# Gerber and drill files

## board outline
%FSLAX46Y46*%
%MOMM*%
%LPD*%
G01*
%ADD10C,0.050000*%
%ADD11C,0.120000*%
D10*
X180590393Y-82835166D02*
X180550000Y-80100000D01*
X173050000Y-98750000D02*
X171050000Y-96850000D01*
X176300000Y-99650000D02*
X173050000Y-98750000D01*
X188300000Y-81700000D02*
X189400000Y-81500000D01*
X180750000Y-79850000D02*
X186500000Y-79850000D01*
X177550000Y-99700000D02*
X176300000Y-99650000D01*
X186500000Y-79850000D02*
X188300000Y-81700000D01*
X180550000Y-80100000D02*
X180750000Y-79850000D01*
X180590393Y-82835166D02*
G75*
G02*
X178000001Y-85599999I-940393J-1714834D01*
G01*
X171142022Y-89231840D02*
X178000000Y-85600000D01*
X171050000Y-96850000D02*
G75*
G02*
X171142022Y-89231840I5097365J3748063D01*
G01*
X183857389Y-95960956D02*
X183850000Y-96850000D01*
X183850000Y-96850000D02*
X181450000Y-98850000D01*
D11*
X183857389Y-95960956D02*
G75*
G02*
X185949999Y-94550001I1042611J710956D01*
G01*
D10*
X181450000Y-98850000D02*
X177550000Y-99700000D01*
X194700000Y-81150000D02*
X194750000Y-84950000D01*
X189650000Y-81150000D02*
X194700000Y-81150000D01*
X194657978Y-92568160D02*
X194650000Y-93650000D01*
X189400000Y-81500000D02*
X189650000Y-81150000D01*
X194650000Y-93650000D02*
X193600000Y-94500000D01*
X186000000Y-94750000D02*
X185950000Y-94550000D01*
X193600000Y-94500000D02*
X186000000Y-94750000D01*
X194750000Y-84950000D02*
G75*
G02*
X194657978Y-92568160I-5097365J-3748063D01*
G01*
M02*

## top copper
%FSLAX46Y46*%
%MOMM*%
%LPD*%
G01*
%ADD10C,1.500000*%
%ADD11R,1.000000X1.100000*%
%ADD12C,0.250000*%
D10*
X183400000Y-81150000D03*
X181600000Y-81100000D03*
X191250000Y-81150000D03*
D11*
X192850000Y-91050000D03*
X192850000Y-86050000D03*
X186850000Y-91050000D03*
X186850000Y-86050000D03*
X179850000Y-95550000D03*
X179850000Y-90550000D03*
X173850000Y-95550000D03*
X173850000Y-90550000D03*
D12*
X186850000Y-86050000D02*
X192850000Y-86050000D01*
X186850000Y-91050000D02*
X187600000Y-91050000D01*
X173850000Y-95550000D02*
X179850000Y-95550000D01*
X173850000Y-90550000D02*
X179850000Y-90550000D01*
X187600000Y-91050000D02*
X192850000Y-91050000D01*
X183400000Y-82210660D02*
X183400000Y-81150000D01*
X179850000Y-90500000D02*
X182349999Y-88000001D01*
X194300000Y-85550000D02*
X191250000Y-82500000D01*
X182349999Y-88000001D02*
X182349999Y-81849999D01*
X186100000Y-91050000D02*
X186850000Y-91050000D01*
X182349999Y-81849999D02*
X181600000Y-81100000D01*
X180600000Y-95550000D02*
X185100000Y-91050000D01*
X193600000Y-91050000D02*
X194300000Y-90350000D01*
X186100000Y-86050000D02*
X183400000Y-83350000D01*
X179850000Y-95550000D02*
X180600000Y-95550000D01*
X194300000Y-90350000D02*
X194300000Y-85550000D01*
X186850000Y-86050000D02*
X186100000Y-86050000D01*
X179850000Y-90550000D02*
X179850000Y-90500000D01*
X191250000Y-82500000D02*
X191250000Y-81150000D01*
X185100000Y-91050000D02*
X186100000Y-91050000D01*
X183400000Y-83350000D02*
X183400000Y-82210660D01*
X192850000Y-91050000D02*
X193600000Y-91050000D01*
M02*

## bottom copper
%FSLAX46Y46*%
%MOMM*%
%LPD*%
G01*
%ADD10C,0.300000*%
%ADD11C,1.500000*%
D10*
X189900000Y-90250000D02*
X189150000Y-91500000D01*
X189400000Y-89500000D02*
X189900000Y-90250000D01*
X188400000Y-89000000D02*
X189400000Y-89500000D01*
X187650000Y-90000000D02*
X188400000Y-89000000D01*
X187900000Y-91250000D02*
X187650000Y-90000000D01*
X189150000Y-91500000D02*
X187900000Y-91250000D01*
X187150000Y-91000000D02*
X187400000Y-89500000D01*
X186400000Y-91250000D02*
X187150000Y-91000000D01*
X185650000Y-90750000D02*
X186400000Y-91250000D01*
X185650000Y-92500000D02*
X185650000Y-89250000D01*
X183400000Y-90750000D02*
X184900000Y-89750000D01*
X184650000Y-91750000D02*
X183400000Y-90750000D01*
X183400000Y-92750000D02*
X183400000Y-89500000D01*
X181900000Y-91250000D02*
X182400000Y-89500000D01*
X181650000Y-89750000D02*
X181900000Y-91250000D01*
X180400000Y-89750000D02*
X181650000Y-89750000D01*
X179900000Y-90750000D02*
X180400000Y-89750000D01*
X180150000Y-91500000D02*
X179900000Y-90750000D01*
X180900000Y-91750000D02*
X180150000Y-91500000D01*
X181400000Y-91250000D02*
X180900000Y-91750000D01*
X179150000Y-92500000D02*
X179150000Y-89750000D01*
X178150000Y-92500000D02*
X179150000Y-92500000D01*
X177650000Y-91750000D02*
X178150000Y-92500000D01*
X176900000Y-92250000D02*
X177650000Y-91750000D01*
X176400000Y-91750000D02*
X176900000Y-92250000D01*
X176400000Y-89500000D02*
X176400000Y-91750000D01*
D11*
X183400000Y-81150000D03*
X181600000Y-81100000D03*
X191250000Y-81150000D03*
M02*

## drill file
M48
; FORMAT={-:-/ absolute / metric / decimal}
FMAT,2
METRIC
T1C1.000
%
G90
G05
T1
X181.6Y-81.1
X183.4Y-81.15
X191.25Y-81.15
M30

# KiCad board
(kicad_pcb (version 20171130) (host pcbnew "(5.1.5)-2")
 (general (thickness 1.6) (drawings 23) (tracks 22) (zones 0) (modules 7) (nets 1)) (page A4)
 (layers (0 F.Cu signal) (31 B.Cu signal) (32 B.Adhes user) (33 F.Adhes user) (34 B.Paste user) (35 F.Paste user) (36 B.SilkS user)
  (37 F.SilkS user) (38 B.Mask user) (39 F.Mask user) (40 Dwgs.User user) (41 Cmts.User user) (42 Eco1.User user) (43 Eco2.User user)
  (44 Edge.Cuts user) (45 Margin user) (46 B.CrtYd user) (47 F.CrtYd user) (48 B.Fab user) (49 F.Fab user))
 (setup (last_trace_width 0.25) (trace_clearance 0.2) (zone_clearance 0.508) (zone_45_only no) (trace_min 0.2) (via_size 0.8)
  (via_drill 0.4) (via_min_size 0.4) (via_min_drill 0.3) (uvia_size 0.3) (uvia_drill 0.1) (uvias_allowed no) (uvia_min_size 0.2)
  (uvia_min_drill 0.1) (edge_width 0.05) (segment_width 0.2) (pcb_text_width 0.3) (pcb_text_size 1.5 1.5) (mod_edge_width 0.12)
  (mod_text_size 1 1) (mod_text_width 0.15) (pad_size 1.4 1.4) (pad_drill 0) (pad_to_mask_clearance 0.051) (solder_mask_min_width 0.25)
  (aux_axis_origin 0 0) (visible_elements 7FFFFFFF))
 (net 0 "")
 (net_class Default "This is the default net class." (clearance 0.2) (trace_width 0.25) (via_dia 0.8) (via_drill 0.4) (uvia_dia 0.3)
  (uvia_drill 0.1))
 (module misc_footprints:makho (layer B.Cu) (at 182.9 90.75)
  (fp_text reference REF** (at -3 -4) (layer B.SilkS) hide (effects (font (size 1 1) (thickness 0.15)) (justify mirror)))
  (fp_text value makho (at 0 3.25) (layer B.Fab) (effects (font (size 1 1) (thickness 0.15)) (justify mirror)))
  (fp_line (start 7 -0.5) (end 6.25 0.75) (layer B.Cu) (width 0.3))
  (fp_line (start 6.5 -1.25) (end 7 -0.5) (layer B.Cu) (width 0.3))
  (fp_line (start 5.5 -1.75) (end 6.5 -1.25) (layer B.Cu) (width 0.3))
  (fp_line (start 4.75 -0.75) (end 5.5 -1.75) (layer B.Cu) (width 0.3))
  (fp_line (start 5 0.5) (end 4.75 -0.75) (layer B.Cu) (width 0.3))
  (fp_line (start 6.25 0.75) (end 5 0.5) (layer B.Cu) (width 0.3))
  (fp_line (start 4.25 0.25) (end 4.5 -1.25) (layer B.Cu) (width 0.3))
  (fp_line (start 3.5 0.5) (end 4.25 0.25) (layer B.Cu) (width 0.3))
  (fp_line (start 2.75 0) (end 3.5 0.5) (layer B.Cu) (width 0.3))
  (fp_line (start 2.75 1.75) (end 2.75 -1.5) (layer B.Cu) (width 0.3)) (fp_line (start 0.5 0) (end 2 -1) (layer B.Cu) (width 0.3))
  (fp_line (start 1.75 1) (end 0.5 0) (layer B.Cu) (width 0.3))
  (fp_line (start 0.5 2) (end 0.5 -1.25) (layer B.Cu) (width 0.3))
  (fp_line (start -1 0.5) (end -0.5 -1.25) (layer B.Cu) (width 0.3))
  (fp_line (start -1.25 -1) (end -1 0.5) (layer B.Cu) (width 0.3))
  (fp_line (start -2.5 -1) (end -1.25 -1) (layer B.Cu) (width 0.3))
  (fp_line (start -3 0) (end -2.5 -1) (layer B.Cu) (width 0.3))
  (fp_line (start -2.75 0.75) (end -3 0) (layer B.Cu) (width 0.3))
  (fp_line (start -2 1) (end -2.75 0.75) (layer B.Cu) (width 0.3))
  (fp_line (start -1.5 0.5) (end -2 1) (layer B.Cu) (width 0.3))
  (fp_line (start -3.75 1.75) (end -3.75 -1) (layer B.Cu) (width 0.3))
  (fp_line (start -4.75 1.75) (end -3.75 1.75) (layer B.Cu) (width 0.3))
  (fp_line (start -5.25 1) (end -4.75 1.75) (layer B.Cu) (width 0.3))
  (fp_line (start -6 1.5) (end -5.25 1) (layer B.Cu) (width 0.3))
  (fp_line (start -6.5 1) (end -6 1.5) (layer B.Cu) (width 0.3))
  (fp_line (start -6.5 -1.25) (end -6.5 1) (layer B.Cu) (width 0.3)))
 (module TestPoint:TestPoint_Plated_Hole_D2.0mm (layer F.Cu) (at 183.4 81.15)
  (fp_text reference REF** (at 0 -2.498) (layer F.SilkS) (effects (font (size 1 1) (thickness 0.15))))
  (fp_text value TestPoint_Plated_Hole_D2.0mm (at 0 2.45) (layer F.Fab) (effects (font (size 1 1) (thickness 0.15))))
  (pad 1 thru_hole circle (at 0 0) (size 1.5 1.5) (drill 1) (layers *.Cu *.Mask)))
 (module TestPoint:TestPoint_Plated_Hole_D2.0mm (layer F.Cu) (at 181.6 81.1)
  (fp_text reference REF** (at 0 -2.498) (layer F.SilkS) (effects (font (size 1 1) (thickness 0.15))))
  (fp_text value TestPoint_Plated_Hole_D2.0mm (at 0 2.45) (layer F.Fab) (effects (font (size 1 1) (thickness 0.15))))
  (pad 1 thru_hole circle (at 0 0) (size 1.5 1.5) (drill 1) (layers *.Cu *.Mask)))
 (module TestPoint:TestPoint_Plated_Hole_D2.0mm (layer F.Cu) (at 191.25 81.15)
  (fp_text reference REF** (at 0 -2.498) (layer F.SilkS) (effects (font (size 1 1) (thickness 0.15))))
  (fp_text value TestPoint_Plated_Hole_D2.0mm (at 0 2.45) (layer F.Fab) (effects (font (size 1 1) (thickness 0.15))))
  (pad 1 thru_hole circle (at 0 0) (size 1.5 1.5) (drill 1) (layers *.Cu *.Mask)))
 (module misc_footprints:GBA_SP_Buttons (layer F.Cu) (at 189.85 88.55)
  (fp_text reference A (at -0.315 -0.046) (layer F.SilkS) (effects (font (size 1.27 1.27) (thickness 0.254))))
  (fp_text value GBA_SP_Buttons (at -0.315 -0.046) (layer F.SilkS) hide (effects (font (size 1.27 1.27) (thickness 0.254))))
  (pad 4 smd rect (at 3 2.5) (size 1 1.1) (layers F.Cu F.Paste F.Mask))
  (pad 3 smd rect (at 3 -2.5) (size 1 1.1) (layers F.Cu F.Paste F.Mask))
  (pad 2 smd rect (at -3 2.5) (size 1 1.1) (layers F.Cu F.Paste F.Mask))
  (pad 1 smd rect (at -3 -2.5) (size 1 1.1) (layers F.Cu F.Paste F.Mask)))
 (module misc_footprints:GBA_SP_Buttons (layer F.Cu) (at 176.85 93.05)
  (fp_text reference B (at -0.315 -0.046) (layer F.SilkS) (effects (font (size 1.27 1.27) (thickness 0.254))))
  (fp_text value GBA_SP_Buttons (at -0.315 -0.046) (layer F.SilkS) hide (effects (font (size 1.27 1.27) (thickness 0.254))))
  (pad 4 smd rect (at 3 2.5) (size 1 1.1) (layers F.Cu F.Paste F.Mask))
  (pad 3 smd rect (at 3 -2.5) (size 1 1.1) (layers F.Cu F.Paste F.Mask))
  (pad 2 smd rect (at -3 2.5) (size 1 1.1) (layers F.Cu F.Paste F.Mask))
  (pad 1 smd rect (at -3 -2.5) (size 1 1.1) (layers F.Cu F.Paste F.Mask)))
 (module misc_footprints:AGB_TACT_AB (layer F.Cu) (at 182.95 89.65)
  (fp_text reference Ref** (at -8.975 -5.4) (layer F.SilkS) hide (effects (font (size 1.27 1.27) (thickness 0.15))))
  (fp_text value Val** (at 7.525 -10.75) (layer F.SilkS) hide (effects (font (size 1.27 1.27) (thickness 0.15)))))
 (gr_line (start 180.590393 82.835166) (end 180.55 80.1) (layer Edge.Cuts) (width 0.05))
 (gr_line (start 173.05 98.75) (end 171.05 96.85) (layer Edge.Cuts) (width 0.05))
 (gr_line (start 176.3 99.65) (end 173.05 98.75) (layer Edge.Cuts) (width 0.05))
 (gr_line (start 188.3 81.7) (end 189.4 81.5) (layer Edge.Cuts) (width 0.05))
 (gr_line (start 180.75 79.85) (end 186.5 79.85) (layer Edge.Cuts) (width 0.05))
 (gr_line (start 177.55 99.7) (end 176.3 99.65) (layer Edge.Cuts) (width 0.05))
 (gr_line (start 186.5 79.85) (end 188.3 81.7) (layer Edge.Cuts) (width 0.05))
 (gr_line (start 180.55 80.1) (end 180.75 79.85) (layer Edge.Cuts) (width 0.05))
 (gr_arc (start 179.65 84.55) (end 178.000001 85.599999) (angle -208.7890124) (layer Edge.Cuts) (width 0.05))
 (gr_line (start 171.142022 89.23184) (end 178 85.6) (layer Edge.Cuts) (width 0.05))
 (gr_arc (start 176.147365 93.101937) (end 171.142022 89.23184) (angle -74.03777643) (layer Edge.Cuts) (width 0.05))
 (gr_line (start 183.857389 95.960956) (end 183.85 96.85) (layer Edge.Cuts) (width 0.05))
 (gr_line (start 183.85 96.85) (end 181.45 98.85) (layer Edge.Cuts) (width 0.05))
 (gr_arc (start 184.9 95.25) (end 185.949999 94.550001) (angle -180.6000055) (layer Edge.Cuts) (width 0.12))
 (gr_line (start 181.45 98.85) (end 177.55 99.7) (layer Edge.Cuts) (width 0.05))
 (gr_line (start 194.7 81.15) (end 194.75 84.95) (layer Edge.Cuts) (width 0.05))
 (gr_line (start 189.65 81.15) (end 194.7 81.15) (layer Edge.Cuts) (width 0.05))
 (gr_line (start 194.657978 92.56816) (end 194.65 93.65) (layer Edge.Cuts) (width 0.05))
 (gr_line (start 189.4 81.5) (end 189.65 81.15) (layer Edge.Cuts) (width 0.05))
 (gr_line (start 194.65 93.65) (end 193.6 94.5) (layer Edge.Cuts) (width 0.05))
 (gr_line (start 186 94.75) (end 185.95 94.55) (layer Edge.Cuts) (width 0.05))
 (gr_line (start 193.6 94.5) (end 186 94.75) (layer Edge.Cuts) (width 0.05))
 (gr_arc (start 189.652635 88.698063) (end 194.657978 92.56816) (angle -74.03777643) (layer Edge.Cuts) (width 0.05))
 (segment (start 186.85 86.05) (end 192.85 86.05) (width 0.25) (layer F.Cu) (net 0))
 (segment (start 186.85 91.05) (end 187.6 91.05) (width 0.25) (layer F.Cu) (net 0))
 (segment (start 173.85 95.55) (end 179.85 95.55) (width 0.25) (layer F.Cu) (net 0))
 (segment (start 173.85 90.55) (end 179.85 90.55) (width 0.25) (layer F.Cu) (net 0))
 (segment (start 187.6 91.05) (end 192.85 91.05) (width 0.25) (layer F.Cu) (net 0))
 (segment (start 183.4 82.21066) (end 183.4 81.15) (width 0.25) (layer F.Cu) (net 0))
 (segment (start 179.85 90.5) (end 182.349999 88.000001) (width 0.25) (layer F.Cu) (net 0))
 (segment (start 194.3 85.55) (end 191.25 82.5) (width 0.25) (layer F.Cu) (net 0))
 (segment (start 182.349999 88.000001) (end 182.349999 81.849999) (width 0.25) (layer F.Cu) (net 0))
 (segment (start 186.1 91.05) (end 186.85 91.05) (width 0.25) (layer F.Cu) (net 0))
 (segment (start 182.349999 81.849999) (end 181.6 81.1) (width 0.25) (layer F.Cu) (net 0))
 (segment (start 180.6 95.55) (end 185.1 91.05) (width 0.25) (layer F.Cu) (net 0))
 (segment (start 193.6 91.05) (end 194.3 90.35) (width 0.25) (layer F.Cu) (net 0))
 (segment (start 186.1 86.05) (end 183.4 83.35) (width 0.25) (layer F.Cu) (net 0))
 (segment (start 179.85 95.55) (end 180.6 95.55) (width 0.25) (layer F.Cu) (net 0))
 (segment (start 194.3 90.35) (end 194.3 85.55) (width 0.25) (layer F.Cu) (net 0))
 (segment (start 186.85 86.05) (end 186.1 86.05) (width 0.25) (layer F.Cu) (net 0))
 (segment (start 179.85 90.55) (end 179.85 90.5) (width 0.25) (layer F.Cu) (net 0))
 (segment (start 191.25 82.5) (end 191.25 81.15) (width 0.25) (layer F.Cu) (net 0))
 (segment (start 185.1 91.05) (end 186.1 91.05) (width 0.25) (layer F.Cu) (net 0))
 (segment (start 183.4 83.35) (end 183.4 82.21066) (width 0.25) (layer F.Cu) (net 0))
 (segment (start 192.85 91.05) (end 193.6 91.05) (width 0.25) (layer F.Cu) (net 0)))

